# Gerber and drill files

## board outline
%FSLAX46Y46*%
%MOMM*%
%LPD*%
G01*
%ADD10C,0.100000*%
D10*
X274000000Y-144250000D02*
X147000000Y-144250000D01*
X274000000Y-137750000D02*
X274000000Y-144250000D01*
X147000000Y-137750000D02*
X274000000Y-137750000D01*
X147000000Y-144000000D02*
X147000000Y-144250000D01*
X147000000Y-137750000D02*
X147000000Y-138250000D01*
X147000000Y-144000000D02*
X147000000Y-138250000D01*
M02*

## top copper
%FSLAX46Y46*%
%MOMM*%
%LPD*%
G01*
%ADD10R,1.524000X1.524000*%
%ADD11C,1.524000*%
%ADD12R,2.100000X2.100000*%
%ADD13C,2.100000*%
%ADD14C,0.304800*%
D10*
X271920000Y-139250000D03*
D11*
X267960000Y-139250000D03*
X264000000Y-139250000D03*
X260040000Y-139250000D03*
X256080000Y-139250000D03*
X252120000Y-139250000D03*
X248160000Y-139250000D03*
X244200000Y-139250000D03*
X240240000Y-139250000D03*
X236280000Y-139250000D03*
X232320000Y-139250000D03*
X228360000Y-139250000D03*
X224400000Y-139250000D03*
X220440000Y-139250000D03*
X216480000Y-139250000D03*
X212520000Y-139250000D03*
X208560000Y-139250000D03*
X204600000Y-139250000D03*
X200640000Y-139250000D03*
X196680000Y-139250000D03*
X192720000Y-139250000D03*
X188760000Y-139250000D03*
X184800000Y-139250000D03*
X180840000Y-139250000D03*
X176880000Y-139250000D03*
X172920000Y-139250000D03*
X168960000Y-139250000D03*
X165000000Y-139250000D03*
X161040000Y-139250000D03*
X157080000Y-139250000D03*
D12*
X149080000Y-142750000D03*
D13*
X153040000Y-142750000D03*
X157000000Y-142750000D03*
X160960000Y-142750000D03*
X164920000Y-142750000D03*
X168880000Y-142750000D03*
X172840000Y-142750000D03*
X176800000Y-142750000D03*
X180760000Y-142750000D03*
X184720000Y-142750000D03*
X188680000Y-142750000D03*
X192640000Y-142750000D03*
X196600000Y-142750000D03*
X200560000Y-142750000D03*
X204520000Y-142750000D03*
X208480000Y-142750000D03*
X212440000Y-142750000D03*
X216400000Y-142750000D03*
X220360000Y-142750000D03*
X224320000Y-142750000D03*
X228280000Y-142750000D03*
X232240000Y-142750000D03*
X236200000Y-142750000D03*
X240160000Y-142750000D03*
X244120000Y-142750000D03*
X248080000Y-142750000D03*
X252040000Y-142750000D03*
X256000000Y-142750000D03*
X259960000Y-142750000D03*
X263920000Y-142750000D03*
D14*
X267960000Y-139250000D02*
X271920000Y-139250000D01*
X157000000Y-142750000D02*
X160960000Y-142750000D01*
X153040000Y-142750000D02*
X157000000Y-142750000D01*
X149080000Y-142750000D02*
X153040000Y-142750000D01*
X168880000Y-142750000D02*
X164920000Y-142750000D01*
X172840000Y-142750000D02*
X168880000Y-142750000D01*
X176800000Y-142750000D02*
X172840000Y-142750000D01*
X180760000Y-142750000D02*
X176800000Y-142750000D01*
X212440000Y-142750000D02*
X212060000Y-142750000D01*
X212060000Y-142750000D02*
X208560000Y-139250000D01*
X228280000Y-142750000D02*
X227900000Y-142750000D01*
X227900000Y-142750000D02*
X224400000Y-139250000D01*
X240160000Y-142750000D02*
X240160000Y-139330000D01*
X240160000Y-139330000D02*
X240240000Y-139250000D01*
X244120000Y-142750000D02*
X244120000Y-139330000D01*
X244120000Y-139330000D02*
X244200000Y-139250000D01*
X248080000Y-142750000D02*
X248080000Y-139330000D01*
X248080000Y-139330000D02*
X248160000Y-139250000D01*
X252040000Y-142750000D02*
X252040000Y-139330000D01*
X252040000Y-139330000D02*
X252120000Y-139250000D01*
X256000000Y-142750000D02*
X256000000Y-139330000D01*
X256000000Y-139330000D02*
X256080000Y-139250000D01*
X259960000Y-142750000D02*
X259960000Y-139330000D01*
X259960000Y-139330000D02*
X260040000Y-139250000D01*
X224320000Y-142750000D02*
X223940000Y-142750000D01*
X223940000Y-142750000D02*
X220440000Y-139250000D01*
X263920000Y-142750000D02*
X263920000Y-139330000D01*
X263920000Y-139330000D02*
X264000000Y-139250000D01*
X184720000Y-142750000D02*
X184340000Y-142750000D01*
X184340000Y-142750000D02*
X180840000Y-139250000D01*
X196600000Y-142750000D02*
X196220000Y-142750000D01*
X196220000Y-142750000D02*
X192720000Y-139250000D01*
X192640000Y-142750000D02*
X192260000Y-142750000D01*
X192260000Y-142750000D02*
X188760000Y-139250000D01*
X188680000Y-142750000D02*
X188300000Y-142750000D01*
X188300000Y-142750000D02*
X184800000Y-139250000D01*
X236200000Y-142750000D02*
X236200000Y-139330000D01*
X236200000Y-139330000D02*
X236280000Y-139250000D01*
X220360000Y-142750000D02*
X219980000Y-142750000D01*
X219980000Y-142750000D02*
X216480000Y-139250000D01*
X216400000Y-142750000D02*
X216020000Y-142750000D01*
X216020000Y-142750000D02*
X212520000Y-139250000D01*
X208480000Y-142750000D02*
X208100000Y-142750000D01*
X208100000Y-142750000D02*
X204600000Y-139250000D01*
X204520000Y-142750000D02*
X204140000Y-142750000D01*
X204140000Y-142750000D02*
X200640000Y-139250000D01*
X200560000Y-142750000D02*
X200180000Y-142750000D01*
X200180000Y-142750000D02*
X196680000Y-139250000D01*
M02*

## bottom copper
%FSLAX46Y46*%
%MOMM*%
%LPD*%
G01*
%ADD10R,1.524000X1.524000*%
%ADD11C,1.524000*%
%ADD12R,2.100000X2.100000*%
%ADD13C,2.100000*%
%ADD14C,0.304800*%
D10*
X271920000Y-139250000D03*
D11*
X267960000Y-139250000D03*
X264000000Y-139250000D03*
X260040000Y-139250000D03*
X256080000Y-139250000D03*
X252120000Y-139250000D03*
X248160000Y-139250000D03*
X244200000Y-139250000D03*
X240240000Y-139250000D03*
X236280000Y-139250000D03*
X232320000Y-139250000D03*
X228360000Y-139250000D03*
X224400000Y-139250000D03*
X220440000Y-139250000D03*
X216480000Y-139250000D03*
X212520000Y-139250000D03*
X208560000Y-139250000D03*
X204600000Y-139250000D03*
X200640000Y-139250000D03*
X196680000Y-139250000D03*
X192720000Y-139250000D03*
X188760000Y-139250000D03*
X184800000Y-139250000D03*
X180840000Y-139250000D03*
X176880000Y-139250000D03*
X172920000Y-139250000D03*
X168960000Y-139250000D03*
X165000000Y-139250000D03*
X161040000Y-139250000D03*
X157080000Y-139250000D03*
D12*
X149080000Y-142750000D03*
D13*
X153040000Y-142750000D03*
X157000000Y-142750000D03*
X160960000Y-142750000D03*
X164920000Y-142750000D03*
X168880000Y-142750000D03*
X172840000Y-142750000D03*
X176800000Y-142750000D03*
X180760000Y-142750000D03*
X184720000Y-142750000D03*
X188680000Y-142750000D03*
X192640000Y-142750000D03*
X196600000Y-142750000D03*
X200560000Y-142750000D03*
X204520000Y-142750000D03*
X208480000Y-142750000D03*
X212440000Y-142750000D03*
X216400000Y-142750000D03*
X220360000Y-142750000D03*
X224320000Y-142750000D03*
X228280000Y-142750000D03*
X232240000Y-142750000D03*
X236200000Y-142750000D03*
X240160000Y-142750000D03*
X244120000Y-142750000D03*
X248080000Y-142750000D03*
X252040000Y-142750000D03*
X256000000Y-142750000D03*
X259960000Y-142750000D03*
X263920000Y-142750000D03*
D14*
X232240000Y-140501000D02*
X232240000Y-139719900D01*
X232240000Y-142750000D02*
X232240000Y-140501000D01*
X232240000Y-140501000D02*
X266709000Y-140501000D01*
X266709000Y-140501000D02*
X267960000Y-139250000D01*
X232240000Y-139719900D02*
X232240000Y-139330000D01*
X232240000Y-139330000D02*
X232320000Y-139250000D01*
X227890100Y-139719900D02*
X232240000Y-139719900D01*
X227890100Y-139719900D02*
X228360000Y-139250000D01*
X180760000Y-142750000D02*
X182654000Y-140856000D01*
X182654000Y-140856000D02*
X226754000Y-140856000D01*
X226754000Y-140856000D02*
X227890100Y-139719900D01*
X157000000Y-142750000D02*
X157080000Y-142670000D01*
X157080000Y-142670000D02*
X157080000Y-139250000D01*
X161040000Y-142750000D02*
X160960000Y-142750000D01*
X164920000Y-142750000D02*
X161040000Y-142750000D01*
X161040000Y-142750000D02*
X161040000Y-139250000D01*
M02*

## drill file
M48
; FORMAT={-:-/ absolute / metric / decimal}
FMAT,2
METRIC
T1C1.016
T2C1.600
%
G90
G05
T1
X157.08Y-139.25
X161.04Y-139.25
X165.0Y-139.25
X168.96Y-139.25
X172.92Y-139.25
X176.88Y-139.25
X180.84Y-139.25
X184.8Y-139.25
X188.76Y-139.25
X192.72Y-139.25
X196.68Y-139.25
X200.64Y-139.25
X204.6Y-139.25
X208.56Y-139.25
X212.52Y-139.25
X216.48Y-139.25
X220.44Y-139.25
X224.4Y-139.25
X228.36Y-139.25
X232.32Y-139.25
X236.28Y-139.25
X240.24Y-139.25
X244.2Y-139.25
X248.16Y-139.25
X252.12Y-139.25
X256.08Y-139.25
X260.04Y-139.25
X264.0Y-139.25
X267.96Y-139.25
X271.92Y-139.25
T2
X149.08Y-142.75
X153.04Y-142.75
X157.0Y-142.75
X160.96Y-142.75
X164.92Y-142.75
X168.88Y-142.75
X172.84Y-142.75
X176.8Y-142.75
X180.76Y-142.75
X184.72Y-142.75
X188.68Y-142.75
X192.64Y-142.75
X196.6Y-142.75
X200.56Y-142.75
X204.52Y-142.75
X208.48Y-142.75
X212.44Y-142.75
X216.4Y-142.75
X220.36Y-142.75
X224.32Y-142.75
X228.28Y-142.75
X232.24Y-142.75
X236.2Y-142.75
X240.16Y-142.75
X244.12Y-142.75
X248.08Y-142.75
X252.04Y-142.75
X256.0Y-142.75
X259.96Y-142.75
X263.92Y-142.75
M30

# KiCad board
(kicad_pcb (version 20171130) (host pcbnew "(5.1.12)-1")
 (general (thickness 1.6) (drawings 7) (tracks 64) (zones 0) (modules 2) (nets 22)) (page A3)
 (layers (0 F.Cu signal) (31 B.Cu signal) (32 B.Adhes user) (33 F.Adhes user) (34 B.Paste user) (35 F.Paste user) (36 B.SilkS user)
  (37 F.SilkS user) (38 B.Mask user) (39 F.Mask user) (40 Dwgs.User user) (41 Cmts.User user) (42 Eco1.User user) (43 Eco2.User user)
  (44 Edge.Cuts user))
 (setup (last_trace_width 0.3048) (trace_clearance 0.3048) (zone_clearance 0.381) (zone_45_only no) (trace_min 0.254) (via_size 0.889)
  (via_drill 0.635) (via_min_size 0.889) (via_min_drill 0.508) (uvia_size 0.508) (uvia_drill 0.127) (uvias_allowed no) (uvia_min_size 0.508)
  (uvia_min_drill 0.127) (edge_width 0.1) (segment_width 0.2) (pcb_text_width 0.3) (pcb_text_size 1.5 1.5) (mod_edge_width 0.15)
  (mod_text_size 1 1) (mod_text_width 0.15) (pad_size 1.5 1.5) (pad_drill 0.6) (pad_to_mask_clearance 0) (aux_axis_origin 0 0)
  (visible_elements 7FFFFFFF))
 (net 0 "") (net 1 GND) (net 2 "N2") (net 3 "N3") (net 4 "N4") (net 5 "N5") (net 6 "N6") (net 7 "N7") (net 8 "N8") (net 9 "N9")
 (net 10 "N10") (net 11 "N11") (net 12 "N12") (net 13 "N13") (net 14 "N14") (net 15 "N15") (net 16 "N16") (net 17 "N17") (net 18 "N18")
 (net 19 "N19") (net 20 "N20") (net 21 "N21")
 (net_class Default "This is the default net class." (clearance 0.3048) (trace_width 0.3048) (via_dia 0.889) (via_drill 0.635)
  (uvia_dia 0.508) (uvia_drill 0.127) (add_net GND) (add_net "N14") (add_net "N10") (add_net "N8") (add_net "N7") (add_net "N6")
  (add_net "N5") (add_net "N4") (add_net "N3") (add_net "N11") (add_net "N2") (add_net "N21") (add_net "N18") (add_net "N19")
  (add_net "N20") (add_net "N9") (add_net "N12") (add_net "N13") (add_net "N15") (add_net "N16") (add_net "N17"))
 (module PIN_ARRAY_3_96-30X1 (layer B.Cu) (at 214.5 139.25 180)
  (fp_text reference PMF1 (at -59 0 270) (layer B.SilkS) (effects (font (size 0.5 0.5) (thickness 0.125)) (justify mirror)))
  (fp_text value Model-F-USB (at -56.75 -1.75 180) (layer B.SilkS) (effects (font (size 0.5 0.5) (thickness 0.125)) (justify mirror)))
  (pad 1 thru_hole rect (at -57.42 0 180) (size 1.524 1.524) (drill 1.016) (layers *.Cu *.Mask B.SilkS) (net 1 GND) (zone_connect 1)
   (thermal_width 0.508) (thermal_gap 0.508))
  (pad 2 thru_hole circle (at -53.46 0 180) (size 1.524 1.524) (drill 1.016) (layers *.Cu *.Mask B.SilkS) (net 1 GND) (zone_connect 1)
   (thermal_width 0.508) (thermal_gap 0.508))
  (pad 3 thru_hole circle (at -49.5 0 180) (size 1.524 1.524) (drill 1.016) (layers *.Cu *.Mask B.SilkS) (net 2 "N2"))
  (pad 4 thru_hole circle (at -45.54 0 180) (size 1.524 1.524) (drill 1.016) (layers *.Cu *.Mask B.SilkS) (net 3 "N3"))
  (pad 5 thru_hole circle (at -41.58 0 180) (size 1.524 1.524) (drill 1.016) (layers *.Cu *.Mask B.SilkS) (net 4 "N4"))
  (pad 6 thru_hole circle (at -37.62 0 180) (size 1.524 1.524) (drill 1.016) (layers *.Cu *.Mask B.SilkS) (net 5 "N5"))
  (pad 7 thru_hole circle (at -33.66 0 180) (size 1.524 1.524) (drill 1.016) (layers *.Cu *.Mask B.SilkS) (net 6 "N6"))
  (pad 8 thru_hole circle (at -29.7 0 180) (size 1.524 1.524) (drill 1.016) (layers *.Cu *.Mask B.SilkS) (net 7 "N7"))
  (pad 9 thru_hole circle (at -25.74 0 180) (size 1.524 1.524) (drill 1.016) (layers *.Cu *.Mask B.SilkS) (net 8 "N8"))
  (pad 10 thru_hole circle (at -21.78 0 180) (size 1.524 1.524) (drill 1.016) (layers *.Cu *.Mask B.SilkS) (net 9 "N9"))
  (pad 11 thru_hole circle (at -17.82 0 180) (size 1.524 1.524) (drill 1.016) (layers *.Cu *.Mask B.SilkS) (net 1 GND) (zone_connect 1)
   (thermal_width 0.508) (thermal_gap 0.508))
  (pad 12 thru_hole circle (at -13.86 0 180) (size 1.524 1.524) (drill 1.016) (layers *.Cu *.Mask B.SilkS) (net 1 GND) (zone_connect 1)
   (thermal_width 0.508) (thermal_gap 0.508))
  (pad 13 thru_hole circle (at -9.9 0 180) (size 1.524 1.524) (drill 1.016) (layers *.Cu *.Mask B.SilkS) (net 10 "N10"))
  (pad 14 thru_hole circle (at -5.94 0 180) (size 1.524 1.524) (drill 1.016) (layers *.Cu *.Mask B.SilkS) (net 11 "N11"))
  (pad 15 thru_hole circle (at -1.98 0 180) (size 1.524 1.524) (drill 1.016) (layers *.Cu *.Mask B.SilkS) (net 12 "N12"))
  (pad 16 thru_hole circle (at 1.98 0 180) (size 1.524 1.524) (drill 1.016) (layers *.Cu *.Mask B.SilkS) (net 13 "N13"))
  (pad 17 thru_hole circle (at 5.94 0 180) (size 1.524 1.524) (drill 1.016) (layers *.Cu *.Mask B.SilkS) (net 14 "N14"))
  (pad 18 thru_hole circle (at 9.9 0 180) (size 1.524 1.524) (drill 1.016) (layers *.Cu *.Mask B.SilkS) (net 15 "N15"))
  (pad 19 thru_hole circle (at 13.86 0 180) (size 1.524 1.524) (drill 1.016) (layers *.Cu *.Mask B.SilkS) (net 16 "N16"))
  (pad 20 thru_hole circle (at 17.82 0 180) (size 1.524 1.524) (drill 1.016) (layers *.Cu *.Mask B.SilkS) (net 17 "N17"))
  (pad 21 thru_hole circle (at 21.78 0 180) (size 1.524 1.524) (drill 1.016) (layers *.Cu *.Mask B.SilkS) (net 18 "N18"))
  (pad 22 thru_hole circle (at 25.74 0 180) (size 1.524 1.524) (drill 1.016) (layers *.Cu *.Mask B.SilkS) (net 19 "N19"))
  (pad 23 thru_hole circle (at 29.7 0 180) (size 1.524 1.524) (drill 1.016) (layers *.Cu *.Mask B.SilkS) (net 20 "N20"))
  (pad 24 thru_hole circle (at 33.66 0 180) (size 1.524 1.524) (drill 1.016) (layers *.Cu *.Mask B.SilkS) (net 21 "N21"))
  (pad 25 thru_hole circle (at 37.62 0 180) (size 1.524 1.524) (drill 1.016) (layers *.Cu *.Mask B.SilkS))
  (pad 26 thru_hole circle (at 41.58 0 180) (size 1.524 1.524) (drill 1.016) (layers *.Cu *.Mask B.SilkS))
  (pad 27 thru_hole circle (at 45.54 0 180) (size 1.524 1.524) (drill 1.016) (layers *.Cu *.Mask B.SilkS))
  (pad 28 thru_hole circle (at 49.5 0 180) (size 1.524 1.524) (drill 1.016) (layers *.Cu *.Mask B.SilkS))
  (pad 29 thru_hole circle (at 53.46 0 180) (size 1.524 1.524) (drill 1.016) (layers *.Cu *.Mask B.SilkS) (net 1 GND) (zone_connect 1)
   (thermal_width 0.508) (thermal_gap 0.508))
  (pad 30 thru_hole circle (at 57.42 0 180) (size 1.524 1.524) (drill 1.016) (layers *.Cu *.Mask B.SilkS) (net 1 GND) (zone_connect 1)
   (thermal_width 0.508) (thermal_gap 0.508)))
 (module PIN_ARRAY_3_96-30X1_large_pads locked (layer F.Cu) (at 206.5 142.75)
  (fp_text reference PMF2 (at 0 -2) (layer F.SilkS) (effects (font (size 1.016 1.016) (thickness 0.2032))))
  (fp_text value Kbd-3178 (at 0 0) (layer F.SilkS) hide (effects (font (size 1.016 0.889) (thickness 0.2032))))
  (pad 1 thru_hole rect (at -57.42 0) (size 2.1 2.1) (drill 1.6) (layers *.Cu *.Mask F.SilkS) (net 1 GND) (zone_connect 1)
   (thermal_width 0.508) (thermal_gap 0.508))
  (pad 2 thru_hole circle (at -53.46 0) (size 2.1 2.1) (drill 1.6) (layers *.Cu *.Mask F.SilkS) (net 1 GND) (zone_connect 1)
   (thermal_width 0.508) (thermal_gap 0.508))
  (pad 3 thru_hole circle (at -49.5 0) (size 2.1 2.1) (drill 1.6) (layers *.Cu *.Mask F.SilkS) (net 1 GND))
  (pad 4 thru_hole circle (at -45.54 0) (size 2.1 2.1) (drill 1.6) (layers *.Cu *.Mask F.SilkS) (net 1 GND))
  (pad 5 thru_hole circle (at -41.58 0) (size 2.1 2.1) (drill 1.6) (layers *.Cu *.Mask F.SilkS) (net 1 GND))
  (pad 6 thru_hole circle (at -37.62 0) (size 2.1 2.1) (drill 1.6) (layers *.Cu *.Mask F.SilkS) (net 1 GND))
  (pad 7 thru_hole circle (at -33.66 0) (size 2.1 2.1) (drill 1.6) (layers *.Cu *.Mask F.SilkS) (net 1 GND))
  (pad 8 thru_hole circle (at -29.7 0) (size 2.1 2.1) (drill 1.6) (layers *.Cu *.Mask F.SilkS) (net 1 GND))
  (pad 9 thru_hole circle (at -25.74 0) (size 2.1 2.1) (drill 1.6) (layers *.Cu *.Mask F.SilkS) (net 1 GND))
  (pad 10 thru_hole circle (at -21.78 0) (size 2.1 2.1) (drill 1.6) (layers *.Cu *.Mask F.SilkS) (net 21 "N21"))
  (pad 11 thru_hole circle (at -17.82 0) (size 2.1 2.1) (drill 1.6) (layers *.Cu *.Mask F.SilkS) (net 20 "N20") (zone_connect 1)
   (thermal_width 0.508) (thermal_gap 0.508))
  (pad 12 thru_hole circle (at -13.86 0) (size 2.1 2.1) (drill 1.6) (layers *.Cu *.Mask F.SilkS) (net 19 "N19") (zone_connect 1)
   (thermal_width 0.508) (thermal_gap 0.508))
  (pad 13 thru_hole circle (at -9.9 0) (size 2.1 2.1) (drill 1.6) (layers *.Cu *.Mask F.SilkS) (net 18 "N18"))
  (pad 14 thru_hole circle (at -5.94 0) (size 2.1 2.1) (drill 1.6) (layers *.Cu *.Mask F.SilkS) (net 17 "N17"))
  (pad 15 thru_hole circle (at -1.98 0) (size 2.1 2.1) (drill 1.6) (layers *.Cu *.Mask F.SilkS) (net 16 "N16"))
  (pad 16 thru_hole circle (at 1.98 0) (size 2.1 2.1) (drill 1.6) (layers *.Cu *.Mask F.SilkS) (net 15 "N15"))
  (pad 17 thru_hole circle (at 5.94 0) (size 2.1 2.1) (drill 1.6) (layers *.Cu *.Mask F.SilkS) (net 14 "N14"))
  (pad 18 thru_hole circle (at 9.9 0) (size 2.1 2.1) (drill 1.6) (layers *.Cu *.Mask F.SilkS) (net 13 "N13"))
  (pad 19 thru_hole circle (at 13.86 0) (size 2.1 2.1) (drill 1.6) (layers *.Cu *.Mask F.SilkS) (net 12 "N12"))
  (pad 20 thru_hole circle (at 17.82 0) (size 2.1 2.1) (drill 1.6) (layers *.Cu *.Mask F.SilkS) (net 11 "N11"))
  (pad 21 thru_hole circle (at 21.78 0) (size 2.1 2.1) (drill 1.6) (layers *.Cu *.Mask F.SilkS) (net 10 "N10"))
  (pad 22 thru_hole circle (at 25.74 0) (size 2.1 2.1) (drill 1.6) (layers *.Cu *.Mask F.SilkS) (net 1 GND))
  (pad 23 thru_hole circle (at 29.7 0) (size 2.1 2.1) (drill 1.6) (layers *.Cu *.Mask F.SilkS) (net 9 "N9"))
  (pad 24 thru_hole circle (at 33.66 0) (size 2.1 2.1) (drill 1.6) (layers *.Cu *.Mask F.SilkS) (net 8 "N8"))
  (pad 25 thru_hole circle (at 37.62 0) (size 2.1 2.1) (drill 1.6) (layers *.Cu *.Mask F.SilkS) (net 7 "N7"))
  (pad 26 thru_hole circle (at 41.58 0) (size 2.1 2.1) (drill 1.6) (layers *.Cu *.Mask F.SilkS) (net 6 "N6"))
  (pad 27 thru_hole circle (at 45.54 0) (size 2.1 2.1) (drill 1.6) (layers *.Cu *.Mask F.SilkS) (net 5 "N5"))
  (pad 28 thru_hole circle (at 49.5 0) (size 2.1 2.1) (drill 1.6) (layers *.Cu *.Mask F.SilkS) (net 4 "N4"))
  (pad 29 thru_hole circle (at 53.46 0) (size 2.1 2.1) (drill 1.6) (layers *.Cu *.Mask F.SilkS) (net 3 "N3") (zone_connect 1)
   (thermal_width 0.508) (thermal_gap 0.508))
  (pad 30 thru_hole circle (at 57.42 0) (size 2.1 2.1) (drill 1.6) (layers *.Cu *.Mask F.SilkS) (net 2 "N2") (zone_connect 1)
   (thermal_width 0.508) (thermal_gap 0.508)))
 (gr_line (start 274 144.25) (end 147 144.25) (angle 90) (layer Edge.Cuts) (width 0.1))
 (gr_line (start 274 137.75) (end 274 144.25) (angle 90) (layer Edge.Cuts) (width 0.1))
 (gr_line (start 147 137.75) (end 274 137.75) (angle 90) (layer Edge.Cuts) (width 0.1))
 (gr_line (start 147 144) (end 147 144.25) (angle 90) (layer Edge.Cuts) (width 0.1))
 (gr_line (start 147 137.75) (end 147 138.25) (angle 90) (layer Edge.Cuts) (width 0.1))
 (gr_line (start 147 144) (end 147 138.25) (angle 90) (layer Edge.Cuts) (width 0.1))
 (segment (start 267.96 139.25) (end 271.92 139.25) (width 0.3048) (layer F.Cu) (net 1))
 (segment (start 232.24 140.501) (end 232.24 139.7199) (width 0.3048) (layer B.Cu) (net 1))
 (segment (start 232.24 142.75) (end 232.24 140.501) (width 0.3048) (layer B.Cu) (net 1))
 (segment (start 232.24 140.501) (end 266.709 140.501) (width 0.3048) (layer B.Cu) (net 1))
 (segment (start 266.709 140.501) (end 267.96 139.25) (width 0.3048) (layer B.Cu) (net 1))
 (segment (start 232.24 139.7199) (end 232.24 139.33) (width 0.3048) (layer B.Cu) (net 1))
 (segment (start 232.24 139.33) (end 232.32 139.25) (width 0.3048) (layer B.Cu) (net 1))
 (segment (start 227.8901 139.7199) (end 232.24 139.7199) (width 0.3048) (layer B.Cu) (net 1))
 (segment (start 227.8901 139.7199) (end 228.36 139.25) (width 0.3048) (layer B.Cu) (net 1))
 (segment (start 180.76 142.75) (end 182.654 140.856) (width 0.3048) (layer B.Cu) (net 1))
 (segment (start 182.654 140.856) (end 226.754 140.856) (width 0.3048) (layer B.Cu) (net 1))
 (segment (start 226.754 140.856) (end 227.8901 139.7199) (width 0.3048) (layer B.Cu) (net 1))
 (segment (start 157 142.75) (end 160.96 142.75) (width 0.3048) (layer F.Cu) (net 1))
 (segment (start 153.04 142.75) (end 157 142.75) (width 0.3048) (layer F.Cu) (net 1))
 (segment (start 149.08 142.75) (end 153.04 142.75) (width 0.3048) (layer F.Cu) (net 1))
 (segment (start 157 142.75) (end 157.08 142.67) (width 0.3048) (layer B.Cu) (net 1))
 (segment (start 157.08 142.67) (end 157.08 139.25) (width 0.3048) (layer B.Cu) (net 1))
 (segment (start 161.04 142.75) (end 160.96 142.75) (width 0.3048) (layer B.Cu) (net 1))
 (segment (start 164.92 142.75) (end 161.04 142.75) (width 0.3048) (layer B.Cu) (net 1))
 (segment (start 161.04 142.75) (end 161.04 139.25) (width 0.3048) (layer B.Cu) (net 1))
 (segment (start 168.88 142.75) (end 164.92 142.75) (width 0.3048) (layer F.Cu) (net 1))
 (segment (start 172.84 142.75) (end 168.88 142.75) (width 0.3048) (layer F.Cu) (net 1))
 (segment (start 176.8 142.75) (end 172.84 142.75) (width 0.3048) (layer F.Cu) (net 1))
 (segment (start 180.76 142.75) (end 176.8 142.75) (width 0.3048) (layer F.Cu) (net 1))
 (segment (start 212.44 142.75) (end 212.06 142.75) (width 0.3048) (layer F.Cu) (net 14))
 (segment (start 212.06 142.75) (end 208.56 139.25) (width 0.3048) (layer F.Cu) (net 14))
 (segment (start 228.28 142.75) (end 227.9 142.75) (width 0.3048) (layer F.Cu) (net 10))
 (segment (start 227.9 142.75) (end 224.4 139.25) (width 0.3048) (layer F.Cu) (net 10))
 (segment (start 240.16 142.75) (end 240.16 139.33) (width 0.3048) (layer F.Cu) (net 8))
 (segment (start 240.16 139.33) (end 240.24 139.25) (width 0.3048) (layer F.Cu) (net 8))
 (segment (start 244.12 142.75) (end 244.12 139.33) (width 0.3048) (layer F.Cu) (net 7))
 (segment (start 244.12 139.33) (end 244.2 139.25) (width 0.3048) (layer F.Cu) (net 7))
 (segment (start 248.08 142.75) (end 248.08 139.33) (width 0.3048) (layer F.Cu) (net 6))
 (segment (start 248.08 139.33) (end 248.16 139.25) (width 0.3048) (layer F.Cu) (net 6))
 (segment (start 252.04 142.75) (end 252.04 139.33) (width 0.3048) (layer F.Cu) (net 5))
 (segment (start 252.04 139.33) (end 252.12 139.25) (width 0.3048) (layer F.Cu) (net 5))
 (segment (start 256 142.75) (end 256 139.33) (width 0.3048) (layer F.Cu) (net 4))
 (segment (start 256 139.33) (end 256.08 139.25) (width 0.3048) (layer F.Cu) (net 4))
 (segment (start 259.96 142.75) (end 259.96 139.33) (width 0.3048) (layer F.Cu) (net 3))
 (segment (start 259.96 139.33) (end 260.04 139.25) (width 0.3048) (layer F.Cu) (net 3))
 (segment (start 224.32 142.75) (end 223.94 142.75) (width 0.3048) (layer F.Cu) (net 11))
 (segment (start 223.94 142.75) (end 220.44 139.25) (width 0.3048) (layer F.Cu) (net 11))
 (segment (start 263.92 142.75) (end 263.92 139.33) (width 0.3048) (layer F.Cu) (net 2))
 (segment (start 263.92 139.33) (end 264 139.25) (width 0.3048) (layer F.Cu) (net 2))
 (segment (start 184.72 142.75) (end 184.34 142.75) (width 0.3048) (layer F.Cu) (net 21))
 (segment (start 184.34 142.75) (end 180.84 139.25) (width 0.3048) (layer F.Cu) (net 21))
 (segment (start 196.6 142.75) (end 196.22 142.75) (width 0.3048) (layer F.Cu) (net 18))
 (segment (start 196.22 142.75) (end 192.72 139.25) (width 0.3048) (layer F.Cu) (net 18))
 (segment (start 192.64 142.75) (end 192.26 142.75) (width 0.3048) (layer F.Cu) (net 19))
 (segment (start 192.26 142.75) (end 188.76 139.25) (width 0.3048) (layer F.Cu) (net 19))
 (segment (start 188.68 142.75) (end 188.3 142.75) (width 0.3048) (layer F.Cu) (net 20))
 (segment (start 188.3 142.75) (end 184.8 139.25) (width 0.3048) (layer F.Cu) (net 20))
 (segment (start 236.2 142.75) (end 236.2 139.33) (width 0.3048) (layer F.Cu) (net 9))
 (segment (start 236.2 139.33) (end 236.28 139.25) (width 0.3048) (layer F.Cu) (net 9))
 (segment (start 220.36 142.75) (end 219.98 142.75) (width 0.3048) (layer F.Cu) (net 12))
 (segment (start 219.98 142.75) (end 216.48 139.25) (width 0.3048) (layer F.Cu) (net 12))
 (segment (start 216.4 142.75) (end 216.02 142.75) (width 0.3048) (layer F.Cu) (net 13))
 (segment (start 216.02 142.75) (end 212.52 139.25) (width 0.3048) (layer F.Cu) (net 13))
 (segment (start 208.48 142.75) (end 208.1 142.75) (width 0.3048) (layer F.Cu) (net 15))
 (segment (start 208.1 142.75) (end 204.6 139.25) (width 0.3048) (layer F.Cu) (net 15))
 (segment (start 204.52 142.75) (end 204.14 142.75) (width 0.3048) (layer F.Cu) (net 16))
 (segment (start 204.14 142.75) (end 200.64 139.25) (width 0.3048) (layer F.Cu) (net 16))
 (segment (start 200.56 142.75) (end 200.18 142.75) (width 0.3048) (layer F.Cu) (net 17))
 (segment (start 200.18 142.75) (end 196.68 139.25) (width 0.3048) (layer F.Cu) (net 17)))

